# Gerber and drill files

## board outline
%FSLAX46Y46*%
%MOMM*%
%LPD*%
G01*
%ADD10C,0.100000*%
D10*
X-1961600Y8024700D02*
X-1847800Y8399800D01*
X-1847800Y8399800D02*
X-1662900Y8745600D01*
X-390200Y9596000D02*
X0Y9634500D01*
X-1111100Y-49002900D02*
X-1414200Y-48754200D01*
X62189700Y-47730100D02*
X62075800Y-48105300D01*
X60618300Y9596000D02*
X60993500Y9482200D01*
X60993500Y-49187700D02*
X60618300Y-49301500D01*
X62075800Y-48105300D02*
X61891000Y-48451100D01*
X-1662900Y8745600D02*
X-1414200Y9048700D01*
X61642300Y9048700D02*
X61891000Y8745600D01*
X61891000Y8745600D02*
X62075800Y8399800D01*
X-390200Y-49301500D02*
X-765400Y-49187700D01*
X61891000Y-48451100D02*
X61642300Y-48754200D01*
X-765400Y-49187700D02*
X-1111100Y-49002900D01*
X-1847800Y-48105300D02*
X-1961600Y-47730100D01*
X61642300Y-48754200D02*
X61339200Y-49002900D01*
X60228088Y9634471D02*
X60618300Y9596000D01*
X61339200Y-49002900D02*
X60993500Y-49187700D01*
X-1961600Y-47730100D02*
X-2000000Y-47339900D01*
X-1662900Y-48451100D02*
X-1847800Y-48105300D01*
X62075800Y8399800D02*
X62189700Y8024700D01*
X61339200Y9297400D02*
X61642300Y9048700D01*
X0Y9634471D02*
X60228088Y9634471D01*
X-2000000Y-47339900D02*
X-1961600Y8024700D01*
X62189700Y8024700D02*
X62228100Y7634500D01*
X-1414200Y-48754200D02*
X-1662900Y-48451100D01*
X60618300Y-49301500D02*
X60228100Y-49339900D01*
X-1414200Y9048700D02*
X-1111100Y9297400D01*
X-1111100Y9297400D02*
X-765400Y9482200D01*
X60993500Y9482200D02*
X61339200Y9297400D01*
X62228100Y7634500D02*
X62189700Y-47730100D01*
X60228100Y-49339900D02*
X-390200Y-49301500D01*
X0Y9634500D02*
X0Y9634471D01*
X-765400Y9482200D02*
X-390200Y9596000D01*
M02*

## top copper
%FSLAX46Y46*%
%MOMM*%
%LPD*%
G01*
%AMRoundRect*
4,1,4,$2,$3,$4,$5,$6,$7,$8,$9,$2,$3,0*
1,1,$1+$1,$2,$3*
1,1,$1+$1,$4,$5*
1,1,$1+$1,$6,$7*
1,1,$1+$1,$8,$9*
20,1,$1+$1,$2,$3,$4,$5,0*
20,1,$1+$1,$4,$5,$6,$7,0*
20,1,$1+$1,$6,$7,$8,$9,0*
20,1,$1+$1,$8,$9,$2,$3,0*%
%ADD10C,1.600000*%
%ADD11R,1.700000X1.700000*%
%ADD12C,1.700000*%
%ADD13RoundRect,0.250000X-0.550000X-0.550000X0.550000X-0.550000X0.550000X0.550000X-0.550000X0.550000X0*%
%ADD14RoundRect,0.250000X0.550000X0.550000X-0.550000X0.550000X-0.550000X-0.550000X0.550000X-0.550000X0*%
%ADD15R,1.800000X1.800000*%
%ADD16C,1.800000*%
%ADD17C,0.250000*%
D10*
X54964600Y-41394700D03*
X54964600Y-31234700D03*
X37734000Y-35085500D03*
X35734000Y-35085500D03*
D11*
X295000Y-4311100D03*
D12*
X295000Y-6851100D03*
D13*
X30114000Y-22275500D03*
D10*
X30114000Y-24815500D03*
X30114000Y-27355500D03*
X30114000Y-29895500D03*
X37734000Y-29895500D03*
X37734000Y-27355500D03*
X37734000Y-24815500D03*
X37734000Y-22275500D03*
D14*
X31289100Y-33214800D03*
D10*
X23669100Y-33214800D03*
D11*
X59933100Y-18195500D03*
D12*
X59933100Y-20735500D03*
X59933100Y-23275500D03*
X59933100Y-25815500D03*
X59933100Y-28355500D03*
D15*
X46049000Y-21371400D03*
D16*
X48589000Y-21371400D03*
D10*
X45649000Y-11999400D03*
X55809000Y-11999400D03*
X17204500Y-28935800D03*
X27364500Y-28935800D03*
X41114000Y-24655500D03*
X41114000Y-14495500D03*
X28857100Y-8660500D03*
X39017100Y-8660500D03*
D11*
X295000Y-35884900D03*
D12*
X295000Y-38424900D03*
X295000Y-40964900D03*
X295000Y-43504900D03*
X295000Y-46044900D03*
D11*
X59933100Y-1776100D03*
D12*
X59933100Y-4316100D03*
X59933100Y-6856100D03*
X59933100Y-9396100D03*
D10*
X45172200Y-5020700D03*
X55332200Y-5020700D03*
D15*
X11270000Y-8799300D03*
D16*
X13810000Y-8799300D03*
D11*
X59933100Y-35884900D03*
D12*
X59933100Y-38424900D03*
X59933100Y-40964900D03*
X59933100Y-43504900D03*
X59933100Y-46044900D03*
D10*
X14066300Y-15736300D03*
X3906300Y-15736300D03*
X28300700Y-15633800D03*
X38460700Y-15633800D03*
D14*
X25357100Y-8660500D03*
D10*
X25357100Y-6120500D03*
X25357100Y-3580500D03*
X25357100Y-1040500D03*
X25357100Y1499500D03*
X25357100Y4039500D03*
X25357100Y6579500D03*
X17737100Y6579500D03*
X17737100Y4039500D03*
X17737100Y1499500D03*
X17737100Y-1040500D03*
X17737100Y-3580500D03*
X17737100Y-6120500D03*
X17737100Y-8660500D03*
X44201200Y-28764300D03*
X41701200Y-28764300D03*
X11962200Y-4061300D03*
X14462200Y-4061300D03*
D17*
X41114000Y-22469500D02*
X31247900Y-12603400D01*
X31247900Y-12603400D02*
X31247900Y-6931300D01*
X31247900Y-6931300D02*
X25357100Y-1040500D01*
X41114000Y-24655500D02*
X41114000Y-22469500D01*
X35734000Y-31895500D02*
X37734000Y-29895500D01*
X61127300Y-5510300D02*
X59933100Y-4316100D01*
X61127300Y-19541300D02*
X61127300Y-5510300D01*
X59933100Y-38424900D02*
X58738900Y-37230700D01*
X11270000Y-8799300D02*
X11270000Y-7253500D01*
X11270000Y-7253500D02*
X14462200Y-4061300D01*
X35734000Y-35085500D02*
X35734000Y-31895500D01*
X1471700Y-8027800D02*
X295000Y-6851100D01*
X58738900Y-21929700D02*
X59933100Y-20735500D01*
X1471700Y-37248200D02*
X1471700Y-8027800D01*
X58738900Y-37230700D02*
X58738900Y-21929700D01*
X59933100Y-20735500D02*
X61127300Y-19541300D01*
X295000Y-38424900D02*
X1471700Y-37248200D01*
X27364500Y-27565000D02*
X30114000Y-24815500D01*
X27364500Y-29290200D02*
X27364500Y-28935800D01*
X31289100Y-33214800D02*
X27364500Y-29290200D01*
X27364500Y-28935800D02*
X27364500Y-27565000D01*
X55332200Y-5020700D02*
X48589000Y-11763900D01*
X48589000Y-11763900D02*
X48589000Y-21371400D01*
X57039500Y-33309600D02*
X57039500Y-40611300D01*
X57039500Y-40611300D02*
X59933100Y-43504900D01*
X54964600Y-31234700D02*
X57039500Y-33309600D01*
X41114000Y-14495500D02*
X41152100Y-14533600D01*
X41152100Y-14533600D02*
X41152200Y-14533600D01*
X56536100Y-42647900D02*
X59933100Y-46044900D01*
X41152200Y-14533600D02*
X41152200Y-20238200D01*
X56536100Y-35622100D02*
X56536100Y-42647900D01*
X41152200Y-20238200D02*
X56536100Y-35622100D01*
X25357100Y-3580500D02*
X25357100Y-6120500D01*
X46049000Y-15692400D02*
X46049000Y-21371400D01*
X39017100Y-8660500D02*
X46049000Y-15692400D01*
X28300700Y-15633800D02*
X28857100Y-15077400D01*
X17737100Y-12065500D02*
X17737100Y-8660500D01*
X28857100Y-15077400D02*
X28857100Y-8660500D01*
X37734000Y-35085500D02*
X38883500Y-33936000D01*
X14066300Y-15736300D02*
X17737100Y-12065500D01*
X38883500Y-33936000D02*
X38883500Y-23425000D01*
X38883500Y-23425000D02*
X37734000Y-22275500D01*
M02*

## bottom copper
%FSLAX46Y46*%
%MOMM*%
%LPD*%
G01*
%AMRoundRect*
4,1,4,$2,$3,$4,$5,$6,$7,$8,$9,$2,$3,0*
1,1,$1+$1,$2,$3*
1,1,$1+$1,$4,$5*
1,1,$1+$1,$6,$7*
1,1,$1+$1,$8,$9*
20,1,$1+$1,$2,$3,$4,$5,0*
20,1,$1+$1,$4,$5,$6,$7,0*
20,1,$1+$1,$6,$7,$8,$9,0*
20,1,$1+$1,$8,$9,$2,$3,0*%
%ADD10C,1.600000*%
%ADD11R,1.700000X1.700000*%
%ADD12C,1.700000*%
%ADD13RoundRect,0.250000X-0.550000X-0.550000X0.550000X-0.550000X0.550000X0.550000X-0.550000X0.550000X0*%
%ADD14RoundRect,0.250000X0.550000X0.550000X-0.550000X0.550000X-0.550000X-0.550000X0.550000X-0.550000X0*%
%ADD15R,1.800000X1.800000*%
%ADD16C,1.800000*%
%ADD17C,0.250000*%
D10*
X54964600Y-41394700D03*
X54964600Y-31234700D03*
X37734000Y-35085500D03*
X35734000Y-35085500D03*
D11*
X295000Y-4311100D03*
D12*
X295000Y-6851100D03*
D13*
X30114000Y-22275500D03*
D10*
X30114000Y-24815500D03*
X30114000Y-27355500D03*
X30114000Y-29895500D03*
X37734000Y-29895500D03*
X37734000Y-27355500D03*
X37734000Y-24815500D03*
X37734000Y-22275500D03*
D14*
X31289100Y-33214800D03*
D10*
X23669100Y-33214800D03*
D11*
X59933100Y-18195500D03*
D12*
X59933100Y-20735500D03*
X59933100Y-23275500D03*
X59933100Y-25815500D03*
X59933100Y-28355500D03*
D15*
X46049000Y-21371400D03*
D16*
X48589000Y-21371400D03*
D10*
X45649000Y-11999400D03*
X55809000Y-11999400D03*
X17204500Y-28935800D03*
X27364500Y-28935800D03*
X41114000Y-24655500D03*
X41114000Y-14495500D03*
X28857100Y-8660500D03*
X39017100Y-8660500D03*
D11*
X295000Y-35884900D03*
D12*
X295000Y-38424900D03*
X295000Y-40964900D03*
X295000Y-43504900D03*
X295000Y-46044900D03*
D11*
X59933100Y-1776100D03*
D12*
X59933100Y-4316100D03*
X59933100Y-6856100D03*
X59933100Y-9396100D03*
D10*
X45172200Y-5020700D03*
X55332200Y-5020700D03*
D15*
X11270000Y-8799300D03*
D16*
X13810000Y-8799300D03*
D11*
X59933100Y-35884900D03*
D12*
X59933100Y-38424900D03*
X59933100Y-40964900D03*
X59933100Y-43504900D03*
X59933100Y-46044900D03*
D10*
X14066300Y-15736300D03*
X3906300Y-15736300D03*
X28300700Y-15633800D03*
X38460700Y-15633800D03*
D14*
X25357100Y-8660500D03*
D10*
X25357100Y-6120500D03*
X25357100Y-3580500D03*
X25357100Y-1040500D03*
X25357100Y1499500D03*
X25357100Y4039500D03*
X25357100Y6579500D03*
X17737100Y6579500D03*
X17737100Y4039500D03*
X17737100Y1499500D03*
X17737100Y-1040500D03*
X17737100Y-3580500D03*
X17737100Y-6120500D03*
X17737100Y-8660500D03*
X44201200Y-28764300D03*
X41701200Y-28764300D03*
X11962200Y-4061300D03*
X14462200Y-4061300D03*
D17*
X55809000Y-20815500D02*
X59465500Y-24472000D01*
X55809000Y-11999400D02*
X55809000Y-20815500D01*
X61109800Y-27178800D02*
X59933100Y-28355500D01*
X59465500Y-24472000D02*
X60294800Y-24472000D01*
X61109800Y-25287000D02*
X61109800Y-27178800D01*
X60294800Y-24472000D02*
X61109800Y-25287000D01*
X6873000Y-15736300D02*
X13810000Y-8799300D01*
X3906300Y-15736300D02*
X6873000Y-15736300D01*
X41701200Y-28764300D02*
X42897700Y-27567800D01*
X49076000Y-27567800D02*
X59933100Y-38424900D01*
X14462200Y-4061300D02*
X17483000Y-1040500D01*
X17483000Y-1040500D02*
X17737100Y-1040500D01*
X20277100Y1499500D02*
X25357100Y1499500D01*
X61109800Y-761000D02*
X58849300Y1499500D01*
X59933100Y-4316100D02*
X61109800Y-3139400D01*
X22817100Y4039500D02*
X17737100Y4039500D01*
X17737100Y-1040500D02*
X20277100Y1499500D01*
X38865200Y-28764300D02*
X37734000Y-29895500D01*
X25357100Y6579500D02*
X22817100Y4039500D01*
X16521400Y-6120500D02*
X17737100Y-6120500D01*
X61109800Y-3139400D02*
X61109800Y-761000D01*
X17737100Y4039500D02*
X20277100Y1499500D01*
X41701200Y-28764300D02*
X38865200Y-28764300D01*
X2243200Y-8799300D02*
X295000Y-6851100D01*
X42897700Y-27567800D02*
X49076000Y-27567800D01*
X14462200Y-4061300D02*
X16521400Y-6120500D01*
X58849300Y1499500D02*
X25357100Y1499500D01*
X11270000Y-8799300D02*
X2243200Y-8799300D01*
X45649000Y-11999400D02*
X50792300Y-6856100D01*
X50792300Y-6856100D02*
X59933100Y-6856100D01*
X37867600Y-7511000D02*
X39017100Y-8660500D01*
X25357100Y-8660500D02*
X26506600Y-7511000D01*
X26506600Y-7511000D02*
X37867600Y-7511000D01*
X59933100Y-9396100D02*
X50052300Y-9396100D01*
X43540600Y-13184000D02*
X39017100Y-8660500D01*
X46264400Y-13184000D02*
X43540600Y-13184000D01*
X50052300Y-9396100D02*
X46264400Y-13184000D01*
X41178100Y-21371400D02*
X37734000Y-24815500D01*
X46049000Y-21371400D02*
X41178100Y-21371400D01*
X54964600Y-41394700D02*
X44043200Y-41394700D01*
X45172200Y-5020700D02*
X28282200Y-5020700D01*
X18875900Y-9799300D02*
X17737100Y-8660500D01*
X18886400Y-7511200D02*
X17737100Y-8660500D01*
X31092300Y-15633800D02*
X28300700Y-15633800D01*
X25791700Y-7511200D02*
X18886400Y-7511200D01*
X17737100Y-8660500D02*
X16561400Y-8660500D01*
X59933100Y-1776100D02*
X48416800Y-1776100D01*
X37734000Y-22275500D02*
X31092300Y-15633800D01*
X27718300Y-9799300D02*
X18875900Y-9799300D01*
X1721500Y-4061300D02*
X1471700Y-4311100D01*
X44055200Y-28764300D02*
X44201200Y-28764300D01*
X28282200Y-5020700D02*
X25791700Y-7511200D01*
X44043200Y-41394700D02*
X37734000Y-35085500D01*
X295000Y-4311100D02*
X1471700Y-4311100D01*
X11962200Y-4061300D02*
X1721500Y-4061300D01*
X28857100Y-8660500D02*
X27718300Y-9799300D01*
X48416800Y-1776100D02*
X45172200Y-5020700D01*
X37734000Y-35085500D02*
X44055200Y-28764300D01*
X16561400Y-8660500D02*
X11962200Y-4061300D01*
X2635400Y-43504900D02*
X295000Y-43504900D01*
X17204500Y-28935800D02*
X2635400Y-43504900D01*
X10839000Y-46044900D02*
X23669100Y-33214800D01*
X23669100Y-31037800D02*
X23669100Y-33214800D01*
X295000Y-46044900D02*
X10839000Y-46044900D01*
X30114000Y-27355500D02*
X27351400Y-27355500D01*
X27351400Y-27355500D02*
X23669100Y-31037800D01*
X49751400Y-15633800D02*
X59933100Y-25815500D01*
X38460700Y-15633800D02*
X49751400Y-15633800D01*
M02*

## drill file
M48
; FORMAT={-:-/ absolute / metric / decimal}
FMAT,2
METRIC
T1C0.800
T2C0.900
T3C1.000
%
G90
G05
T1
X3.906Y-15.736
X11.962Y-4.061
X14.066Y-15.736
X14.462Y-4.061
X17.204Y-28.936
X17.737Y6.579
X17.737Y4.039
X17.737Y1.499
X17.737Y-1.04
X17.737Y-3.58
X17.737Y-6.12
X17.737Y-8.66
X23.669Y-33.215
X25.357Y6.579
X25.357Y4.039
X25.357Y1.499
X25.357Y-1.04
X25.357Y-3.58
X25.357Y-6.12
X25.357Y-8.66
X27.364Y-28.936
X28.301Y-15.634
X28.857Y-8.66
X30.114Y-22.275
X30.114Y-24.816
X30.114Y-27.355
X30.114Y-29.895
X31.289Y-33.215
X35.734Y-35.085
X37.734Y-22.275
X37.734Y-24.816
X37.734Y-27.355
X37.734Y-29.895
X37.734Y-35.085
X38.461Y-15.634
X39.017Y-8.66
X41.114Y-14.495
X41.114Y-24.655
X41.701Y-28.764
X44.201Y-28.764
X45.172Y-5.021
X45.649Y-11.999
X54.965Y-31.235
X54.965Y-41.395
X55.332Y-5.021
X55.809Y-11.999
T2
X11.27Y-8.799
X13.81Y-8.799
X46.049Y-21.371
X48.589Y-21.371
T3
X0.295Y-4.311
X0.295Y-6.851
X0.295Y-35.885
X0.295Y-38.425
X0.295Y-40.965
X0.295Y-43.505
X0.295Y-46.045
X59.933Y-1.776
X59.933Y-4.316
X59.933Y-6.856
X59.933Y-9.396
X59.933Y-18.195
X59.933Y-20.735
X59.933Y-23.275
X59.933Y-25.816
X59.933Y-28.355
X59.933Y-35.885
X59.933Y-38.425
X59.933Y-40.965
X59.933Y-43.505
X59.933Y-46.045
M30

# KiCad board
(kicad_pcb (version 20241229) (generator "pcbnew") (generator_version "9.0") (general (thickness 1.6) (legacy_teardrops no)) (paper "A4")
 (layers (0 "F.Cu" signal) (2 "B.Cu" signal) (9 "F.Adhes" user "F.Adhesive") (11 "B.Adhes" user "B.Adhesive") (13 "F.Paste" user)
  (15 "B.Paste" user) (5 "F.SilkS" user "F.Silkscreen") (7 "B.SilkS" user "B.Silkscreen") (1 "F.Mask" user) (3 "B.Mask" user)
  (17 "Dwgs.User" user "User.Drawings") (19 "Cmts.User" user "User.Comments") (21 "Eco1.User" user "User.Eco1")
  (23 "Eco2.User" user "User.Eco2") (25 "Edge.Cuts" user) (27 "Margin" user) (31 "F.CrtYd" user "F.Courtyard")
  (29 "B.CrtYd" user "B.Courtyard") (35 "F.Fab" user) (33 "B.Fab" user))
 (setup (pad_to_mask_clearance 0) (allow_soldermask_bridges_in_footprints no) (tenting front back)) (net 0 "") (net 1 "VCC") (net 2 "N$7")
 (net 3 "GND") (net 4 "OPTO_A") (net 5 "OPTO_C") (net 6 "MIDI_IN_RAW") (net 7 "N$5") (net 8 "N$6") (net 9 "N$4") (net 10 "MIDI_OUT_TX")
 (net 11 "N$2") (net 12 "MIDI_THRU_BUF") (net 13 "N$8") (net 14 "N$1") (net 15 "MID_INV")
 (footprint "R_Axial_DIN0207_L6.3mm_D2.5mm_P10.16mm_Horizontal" (layer "F.Cu") (at 54.9646 41.3947 90)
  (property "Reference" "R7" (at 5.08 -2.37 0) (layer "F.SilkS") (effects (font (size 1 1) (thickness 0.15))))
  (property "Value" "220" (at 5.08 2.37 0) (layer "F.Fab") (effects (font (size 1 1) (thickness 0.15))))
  (pad "1" thru_hole circle (at 0 0 90) (size 1.6 1.6) (drill 0.8) (layers "*.Cu" "*.Mask") (remove_unused_layers no) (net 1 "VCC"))
  (pad "2" thru_hole circle (at 10.16 0 90) (size 1.6 1.6) (drill 0.8) (layers "*.Cu" "*.Mask") (remove_unused_layers no) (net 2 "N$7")))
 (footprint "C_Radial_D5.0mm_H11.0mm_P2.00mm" (layer "F.Cu") (at 37.734 35.0855 180)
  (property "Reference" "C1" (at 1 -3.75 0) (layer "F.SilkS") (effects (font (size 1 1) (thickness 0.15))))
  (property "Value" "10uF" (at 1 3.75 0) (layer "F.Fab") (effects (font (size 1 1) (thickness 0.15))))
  (pad "1" thru_hole circle (at 0 0 180) (size 1.6 1.6) (drill 0.8) (layers "*.Cu" "*.Mask") (remove_unused_layers no) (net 1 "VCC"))
  (pad "2" thru_hole circle (at 2 0 180) (size 1.6 1.6) (drill 0.8) (layers "*.Cu" "*.Mask") (remove_unused_layers no) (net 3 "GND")))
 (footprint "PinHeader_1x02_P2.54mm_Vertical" (layer "F.Cu") (at 0.295 4.3111)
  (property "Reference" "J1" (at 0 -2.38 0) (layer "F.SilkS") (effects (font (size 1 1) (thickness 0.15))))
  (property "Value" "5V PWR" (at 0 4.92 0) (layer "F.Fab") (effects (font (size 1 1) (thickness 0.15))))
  (pad "1" thru_hole rect (at 0 0) (size 1.7 1.7) (drill 1) (layers "*.Cu" "*.Mask") (remove_unused_layers no) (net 1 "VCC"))
  (pad "2" thru_hole circle (at 0 2.54) (size 1.7 1.7) (drill 1) (layers "*.Cu" "*.Mask") (remove_unused_layers no) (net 3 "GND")))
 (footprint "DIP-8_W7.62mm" (layer "F.Cu") (at 30.114 22.2755)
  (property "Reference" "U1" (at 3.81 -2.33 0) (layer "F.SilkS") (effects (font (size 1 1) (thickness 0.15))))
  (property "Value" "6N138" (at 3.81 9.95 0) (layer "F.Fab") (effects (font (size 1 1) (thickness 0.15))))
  (pad "1" thru_hole roundrect (at 0 0) (size 1.6 1.6) (drill 0.8) (layers "*.Cu" "*.Mask") (remove_unused_layers no)
   (roundrect_rratio 0.15625))
  (pad "2" thru_hole circle (at 0 2.54) (size 1.6 1.6) (drill 0.8) (layers "*.Cu" "*.Mask") (remove_unused_layers no) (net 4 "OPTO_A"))
  (pad "3" thru_hole circle (at 0 5.08) (size 1.6 1.6) (drill 0.8) (layers "*.Cu" "*.Mask") (remove_unused_layers no) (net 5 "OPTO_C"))
  (pad "4" thru_hole circle (at 0 7.62) (size 1.6 1.6) (drill 0.8) (layers "*.Cu" "*.Mask") (remove_unused_layers no))
  (pad "5" thru_hole circle (at 7.62 7.62) (size 1.6 1.6) (drill 0.8) (layers "*.Cu" "*.Mask") (remove_unused_layers no) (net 3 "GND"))
  (pad "6" thru_hole circle (at 7.62 5.08) (size 1.6 1.6) (drill 0.8) (layers "*.Cu" "*.Mask") (remove_unused_layers no))
  (pad "7" thru_hole circle (at 7.62 2.54) (size 1.6 1.6) (drill 0.8) (layers "*.Cu" "*.Mask") (remove_unused_layers no)
   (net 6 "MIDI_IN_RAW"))
  (pad "8" thru_hole circle (at 7.62 0) (size 1.6 1.6) (drill 0.8) (layers "*.Cu" "*.Mask") (remove_unused_layers no) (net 1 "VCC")))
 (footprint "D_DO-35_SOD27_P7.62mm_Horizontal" (layer "F.Cu") (at 31.2891 33.2148 180)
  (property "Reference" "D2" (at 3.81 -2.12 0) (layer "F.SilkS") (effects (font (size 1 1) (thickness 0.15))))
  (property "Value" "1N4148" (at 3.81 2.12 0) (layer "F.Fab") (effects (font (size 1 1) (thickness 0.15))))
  (pad "1" thru_hole roundrect (at 0 0 180) (size 1.6 1.6) (drill 0.8) (layers "*.Cu" "*.Mask") (remove_unused_layers no)
   (roundrect_rratio 0.15625) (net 4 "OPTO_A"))
  (pad "2" thru_hole circle (at 7.62 0 180) (size 1.6 1.6) (drill 0.8) (layers "*.Cu" "*.Mask") (remove_unused_layers no) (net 5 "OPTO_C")))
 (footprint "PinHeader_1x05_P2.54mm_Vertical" (layer "F.Cu") (at 59.9331 18.1955)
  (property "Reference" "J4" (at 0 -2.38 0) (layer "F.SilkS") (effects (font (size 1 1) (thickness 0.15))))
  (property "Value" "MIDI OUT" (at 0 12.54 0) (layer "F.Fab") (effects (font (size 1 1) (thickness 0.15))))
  (pad "1" thru_hole rect (at 0 0) (size 1.7 1.7) (drill 1) (layers "*.Cu" "*.Mask") (remove_unused_layers no))
  (pad "2" thru_hole circle (at 0 2.54) (size 1.7 1.7) (drill 1) (layers "*.Cu" "*.Mask") (remove_unused_layers no) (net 3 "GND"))
  (pad "3" thru_hole circle (at 0 5.08) (size 1.7 1.7) (drill 1) (layers "*.Cu" "*.Mask") (remove_unused_layers no))
  (pad "4" thru_hole circle (at 0 7.62) (size 1.7 1.7) (drill 1) (layers "*.Cu" "*.Mask") (remove_unused_layers no) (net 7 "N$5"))
  (pad "5" thru_hole circle (at 0 10.16) (size 1.7 1.7) (drill 1) (layers "*.Cu" "*.Mask") (remove_unused_layers no) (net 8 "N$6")))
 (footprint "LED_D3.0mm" (layer "F.Cu") (at 46.049 21.3714)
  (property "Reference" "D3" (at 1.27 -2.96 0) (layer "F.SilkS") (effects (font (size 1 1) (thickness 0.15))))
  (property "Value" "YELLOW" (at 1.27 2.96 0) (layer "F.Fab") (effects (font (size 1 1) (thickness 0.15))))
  (pad "1" thru_hole rect (at 0 0) (size 1.8 1.8) (drill 0.9) (layers "*.Cu" "*.Mask") (remove_unused_layers no) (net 6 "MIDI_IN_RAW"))
  (pad "2" thru_hole circle (at 2.54 0) (size 1.8 1.8) (drill 0.9) (layers "*.Cu" "*.Mask") (remove_unused_layers no) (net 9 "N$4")))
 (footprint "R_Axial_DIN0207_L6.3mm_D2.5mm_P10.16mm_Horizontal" (layer "F.Cu") (at 45.649 11.9994)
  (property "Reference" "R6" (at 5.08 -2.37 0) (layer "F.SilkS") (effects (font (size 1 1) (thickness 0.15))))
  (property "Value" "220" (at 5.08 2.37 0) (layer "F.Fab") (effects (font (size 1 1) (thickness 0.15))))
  (pad "1" thru_hole circle (at 0 0) (size 1.6 1.6) (drill 0.8) (layers "*.Cu" "*.Mask") (remove_unused_layers no) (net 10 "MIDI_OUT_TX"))
  (pad "2" thru_hole circle (at 10.16 0) (size 1.6 1.6) (drill 0.8) (layers "*.Cu" "*.Mask") (remove_unused_layers no) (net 8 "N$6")))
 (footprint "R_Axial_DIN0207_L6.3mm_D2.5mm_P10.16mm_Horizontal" (layer "F.Cu") (at 17.2045 28.9358)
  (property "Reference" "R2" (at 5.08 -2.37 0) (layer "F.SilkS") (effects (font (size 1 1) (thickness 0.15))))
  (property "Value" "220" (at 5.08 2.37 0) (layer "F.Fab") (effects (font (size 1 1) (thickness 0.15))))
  (pad "1" thru_hole circle (at 0 0) (size 1.6 1.6) (drill 0.8) (layers "*.Cu" "*.Mask") (remove_unused_layers no) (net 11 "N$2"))
  (pad "2" thru_hole circle (at 10.16 0) (size 1.6 1.6) (drill 0.8) (layers "*.Cu" "*.Mask") (remove_unused_layers no) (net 4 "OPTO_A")))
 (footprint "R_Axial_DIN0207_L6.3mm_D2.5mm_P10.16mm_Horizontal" (layer "F.Cu") (at 41.114 24.6555 90)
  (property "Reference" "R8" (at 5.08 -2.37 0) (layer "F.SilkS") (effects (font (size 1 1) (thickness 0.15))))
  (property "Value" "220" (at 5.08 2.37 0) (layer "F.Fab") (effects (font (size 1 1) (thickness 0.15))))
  (pad "1" thru_hole circle (at 0 0 90) (size 1.6 1.6) (drill 0.8) (layers "*.Cu" "*.Mask") (remove_unused_layers no)
   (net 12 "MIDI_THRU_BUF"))
  (pad "2" thru_hole circle (at 10.16 0 90) (size 1.6 1.6) (drill 0.8) (layers "*.Cu" "*.Mask") (remove_unused_layers no) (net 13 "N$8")))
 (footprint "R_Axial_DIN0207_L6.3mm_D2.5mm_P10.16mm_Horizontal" (layer "F.Cu") (at 28.8571 8.6605)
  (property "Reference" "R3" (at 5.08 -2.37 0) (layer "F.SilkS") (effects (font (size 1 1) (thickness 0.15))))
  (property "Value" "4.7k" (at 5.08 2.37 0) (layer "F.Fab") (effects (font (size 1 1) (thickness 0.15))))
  (pad "1" thru_hole circle (at 0 0) (size 1.6 1.6) (drill 0.8) (layers "*.Cu" "*.Mask") (remove_unused_layers no) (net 1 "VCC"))
  (pad "2" thru_hole circle (at 10.16 0) (size 1.6 1.6) (drill 0.8) (layers "*.Cu" "*.Mask") (remove_unused_layers no) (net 6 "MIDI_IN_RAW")))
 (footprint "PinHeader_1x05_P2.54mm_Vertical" (layer "F.Cu") (at 0.295 35.8849)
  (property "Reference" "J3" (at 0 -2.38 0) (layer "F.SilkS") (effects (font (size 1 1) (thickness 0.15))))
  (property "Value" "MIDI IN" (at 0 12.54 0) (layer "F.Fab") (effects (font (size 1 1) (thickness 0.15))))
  (pad "1" thru_hole rect (at 0 0) (size 1.7 1.7) (drill 1) (layers "*.Cu" "*.Mask") (remove_unused_layers no))
  (pad "2" thru_hole circle (at 0 2.54) (size 1.7 1.7) (drill 1) (layers "*.Cu" "*.Mask") (remove_unused_layers no) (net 3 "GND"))
  (pad "3" thru_hole circle (at 0 5.08) (size 1.7 1.7) (drill 1) (layers "*.Cu" "*.Mask") (remove_unused_layers no))
  (pad "4" thru_hole circle (at 0 7.62) (size 1.7 1.7) (drill 1) (layers "*.Cu" "*.Mask") (remove_unused_layers no) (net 11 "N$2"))
  (pad "5" thru_hole circle (at 0 10.16) (size 1.7 1.7) (drill 1) (layers "*.Cu" "*.Mask") (remove_unused_layers no) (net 5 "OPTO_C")))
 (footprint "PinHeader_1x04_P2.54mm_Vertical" (layer "F.Cu") (at 59.9331 1.7761)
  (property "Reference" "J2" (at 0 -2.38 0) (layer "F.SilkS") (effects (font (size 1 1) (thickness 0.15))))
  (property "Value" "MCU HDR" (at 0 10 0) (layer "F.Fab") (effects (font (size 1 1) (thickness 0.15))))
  (pad "1" thru_hole rect (at 0 0) (size 1.7 1.7) (drill 1) (layers "*.Cu" "*.Mask") (remove_unused_layers no) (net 1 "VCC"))
  (pad "2" thru_hole circle (at 0 2.54) (size 1.7 1.7) (drill 1) (layers "*.Cu" "*.Mask") (remove_unused_layers no) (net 3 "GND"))
  (pad "3" thru_hole circle (at 0 5.08) (size 1.7 1.7) (drill 1) (layers "*.Cu" "*.Mask") (remove_unused_layers no) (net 10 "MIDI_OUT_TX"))
  (pad "4" thru_hole circle (at 0 7.62) (size 1.7 1.7) (drill 1) (layers "*.Cu" "*.Mask") (remove_unused_layers no) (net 6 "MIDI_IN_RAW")))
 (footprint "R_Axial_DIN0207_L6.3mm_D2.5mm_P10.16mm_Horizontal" (layer "F.Cu") (at 45.1722 5.0207)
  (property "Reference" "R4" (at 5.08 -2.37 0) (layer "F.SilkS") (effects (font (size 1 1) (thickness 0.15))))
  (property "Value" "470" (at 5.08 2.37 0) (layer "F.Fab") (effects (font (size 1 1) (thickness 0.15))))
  (pad "1" thru_hole circle (at 0 0) (size 1.6 1.6) (drill 0.8) (layers "*.Cu" "*.Mask") (remove_unused_layers no) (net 1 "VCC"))
  (pad "2" thru_hole circle (at 10.16 0) (size 1.6 1.6) (drill 0.8) (layers "*.Cu" "*.Mask") (remove_unused_layers no) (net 9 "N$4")))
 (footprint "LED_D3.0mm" (layer "F.Cu") (at 11.27 8.7993)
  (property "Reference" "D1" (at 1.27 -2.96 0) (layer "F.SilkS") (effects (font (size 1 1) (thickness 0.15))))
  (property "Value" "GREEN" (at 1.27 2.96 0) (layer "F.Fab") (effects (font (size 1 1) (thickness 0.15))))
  (pad "1" thru_hole rect (at 0 0) (size 1.8 1.8) (drill 0.9) (layers "*.Cu" "*.Mask") (remove_unused_layers no) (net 3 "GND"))
  (pad "2" thru_hole circle (at 2.54 0) (size 1.8 1.8) (drill 0.9) (layers "*.Cu" "*.Mask") (remove_unused_layers no) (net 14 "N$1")))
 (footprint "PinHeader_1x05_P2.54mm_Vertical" (layer "F.Cu") (at 59.9331 35.8849)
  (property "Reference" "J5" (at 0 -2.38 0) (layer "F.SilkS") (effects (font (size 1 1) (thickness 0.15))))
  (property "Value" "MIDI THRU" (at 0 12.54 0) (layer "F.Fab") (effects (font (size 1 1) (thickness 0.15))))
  (pad "1" thru_hole rect (at 0 0) (size 1.7 1.7) (drill 1) (layers "*.Cu" "*.Mask") (remove_unused_layers no))
  (pad "2" thru_hole circle (at 0 2.54) (size 1.7 1.7) (drill 1) (layers "*.Cu" "*.Mask") (remove_unused_layers no) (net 3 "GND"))
  (pad "3" thru_hole circle (at 0 5.08) (size 1.7 1.7) (drill 1) (layers "*.Cu" "*.Mask") (remove_unused_layers no))
  (pad "4" thru_hole circle (at 0 7.62) (size 1.7 1.7) (drill 1) (layers "*.Cu" "*.Mask") (remove_unused_layers no) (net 2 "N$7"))
  (pad "5" thru_hole circle (at 0 10.16) (size 1.7 1.7) (drill 1) (layers "*.Cu" "*.Mask") (remove_unused_layers no) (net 13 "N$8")))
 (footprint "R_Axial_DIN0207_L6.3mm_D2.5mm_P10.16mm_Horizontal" (layer "F.Cu") (at 14.0663 15.7363 180)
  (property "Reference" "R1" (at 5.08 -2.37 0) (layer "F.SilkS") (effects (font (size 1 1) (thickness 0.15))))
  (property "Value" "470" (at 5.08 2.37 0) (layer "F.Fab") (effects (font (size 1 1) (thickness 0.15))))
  (pad "1" thru_hole circle (at 0 0 180) (size 1.6 1.6) (drill 0.8) (layers "*.Cu" "*.Mask") (remove_unused_layers no) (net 1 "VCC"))
  (pad "2" thru_hole circle (at 10.16 0 180) (size 1.6 1.6) (drill 0.8) (layers "*.Cu" "*.Mask") (remove_unused_layers no) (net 14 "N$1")))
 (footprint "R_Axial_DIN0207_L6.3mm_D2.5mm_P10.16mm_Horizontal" (layer "F.Cu") (at 28.3007 15.6338)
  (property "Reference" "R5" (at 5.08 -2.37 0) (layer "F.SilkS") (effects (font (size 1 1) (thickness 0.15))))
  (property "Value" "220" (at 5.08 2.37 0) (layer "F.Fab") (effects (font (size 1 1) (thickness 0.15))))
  (pad "1" thru_hole circle (at 0 0) (size 1.6 1.6) (drill 0.8) (layers "*.Cu" "*.Mask") (remove_unused_layers no) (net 1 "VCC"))
  (pad "2" thru_hole circle (at 10.16 0) (size 1.6 1.6) (drill 0.8) (layers "*.Cu" "*.Mask") (remove_unused_layers no) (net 7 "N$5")))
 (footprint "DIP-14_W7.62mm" (layer "F.Cu") (at 25.3571 8.6605 180)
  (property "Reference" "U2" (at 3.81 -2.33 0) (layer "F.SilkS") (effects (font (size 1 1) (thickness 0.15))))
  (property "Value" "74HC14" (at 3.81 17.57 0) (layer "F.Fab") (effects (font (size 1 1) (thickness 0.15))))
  (pad "1" thru_hole roundrect (at 0 0 180) (size 1.6 1.6) (drill 0.8) (layers "*.Cu" "*.Mask") (remove_unused_layers no)
   (roundrect_rratio 0.15625) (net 6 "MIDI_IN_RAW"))
  (pad "2" thru_hole circle (at 0 2.54 180) (size 1.6 1.6) (drill 0.8) (layers "*.Cu" "*.Mask") (remove_unused_layers no) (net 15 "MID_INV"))
  (pad "3" thru_hole circle (at 0 5.08 180) (size 1.6 1.6) (drill 0.8) (layers "*.Cu" "*.Mask") (remove_unused_layers no) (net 15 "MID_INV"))
  (pad "4" thru_hole circle (at 0 7.62 180) (size 1.6 1.6) (drill 0.8) (layers "*.Cu" "*.Mask") (remove_unused_layers no)
   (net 12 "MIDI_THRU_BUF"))
  (pad "5" thru_hole circle (at 0 10.16 180) (size 1.6 1.6) (drill 0.8) (layers "*.Cu" "*.Mask") (remove_unused_layers no) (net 3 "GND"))
  (pad "6" thru_hole circle (at 0 12.7 180) (size 1.6 1.6) (drill 0.8) (layers "*.Cu" "*.Mask") (remove_unused_layers no))
  (pad "7" thru_hole circle (at 0 15.24 180) (size 1.6 1.6) (drill 0.8) (layers "*.Cu" "*.Mask") (remove_unused_layers no) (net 3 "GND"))
  (pad "8" thru_hole circle (at 7.62 15.24 180) (size 1.6 1.6) (drill 0.8) (layers "*.Cu" "*.Mask") (remove_unused_layers no))
  (pad "9" thru_hole circle (at 7.62 12.7 180) (size 1.6 1.6) (drill 0.8) (layers "*.Cu" "*.Mask") (remove_unused_layers no) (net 3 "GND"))
  (pad "10" thru_hole circle (at 7.62 10.16 180) (size 1.6 1.6) (drill 0.8) (layers "*.Cu" "*.Mask") (remove_unused_layers no))
  (pad "11" thru_hole circle (at 7.62 7.62 180) (size 1.6 1.6) (drill 0.8) (layers "*.Cu" "*.Mask") (remove_unused_layers no) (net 3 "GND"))
  (pad "12" thru_hole circle (at 7.62 5.08 180) (size 1.6 1.6) (drill 0.8) (layers "*.Cu" "*.Mask") (remove_unused_layers no))
  (pad "13" thru_hole circle (at 7.62 2.54 180) (size 1.6 1.6) (drill 0.8) (layers "*.Cu" "*.Mask") (remove_unused_layers no) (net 3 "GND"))
  (pad "14" thru_hole circle (at 7.62 0 180) (size 1.6 1.6) (drill 0.8) (layers "*.Cu" "*.Mask") (remove_unused_layers no) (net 1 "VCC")))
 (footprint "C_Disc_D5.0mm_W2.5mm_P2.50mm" (layer "F.Cu") (at 44.2012 28.7643 180)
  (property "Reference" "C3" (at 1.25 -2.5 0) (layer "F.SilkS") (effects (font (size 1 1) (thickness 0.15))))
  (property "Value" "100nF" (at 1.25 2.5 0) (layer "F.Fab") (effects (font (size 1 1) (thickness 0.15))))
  (pad "1" thru_hole circle (at 0 0 180) (size 1.6 1.6) (drill 0.8) (layers "*.Cu" "*.Mask") (remove_unused_layers no) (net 1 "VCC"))
  (pad "2" thru_hole circle (at 2.5 0 180) (size 1.6 1.6) (drill 0.8) (layers "*.Cu" "*.Mask") (remove_unused_layers no) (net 3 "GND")))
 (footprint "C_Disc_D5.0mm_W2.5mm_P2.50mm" (layer "F.Cu") (at 11.9622 4.0613)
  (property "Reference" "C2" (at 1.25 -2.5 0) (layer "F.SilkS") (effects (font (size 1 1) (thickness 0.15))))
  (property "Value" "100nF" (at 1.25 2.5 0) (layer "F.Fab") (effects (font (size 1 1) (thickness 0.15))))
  (pad "1" thru_hole circle (at 0 0) (size 1.6 1.6) (drill 0.8) (layers "*.Cu" "*.Mask") (remove_unused_layers no) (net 1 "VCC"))
  (pad "2" thru_hole circle (at 2.5 0) (size 1.6 1.6) (drill 0.8) (layers "*.Cu" "*.Mask") (remove_unused_layers no) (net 3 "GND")))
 (gr_line (start -1.9616 -8.0247) (end -1.8478 -8.3998) (stroke (width 0.1) (type solid)) (layer "Edge.Cuts"))
 (gr_line (start -1.8478 -8.3998) (end -1.6629 -8.7456) (stroke (width 0.1) (type solid)) (layer "Edge.Cuts"))
 (gr_line (start -0.3902 -9.596) (end 0 -9.6345) (stroke (width 0.1) (type solid)) (layer "Edge.Cuts"))
 (gr_line (start -1.1111 49.0029) (end -1.4142 48.7542) (stroke (width 0.1) (type solid)) (layer "Edge.Cuts"))
 (gr_line (start 62.1897 47.7301) (end 62.0758 48.1053) (stroke (width 0.1) (type solid)) (layer "Edge.Cuts"))
 (gr_line (start 60.6183 -9.596) (end 60.9935 -9.4822) (stroke (width 0.1) (type solid)) (layer "Edge.Cuts"))
 (gr_line (start 60.9935 49.1877) (end 60.6183 49.3015) (stroke (width 0.1) (type solid)) (layer "Edge.Cuts"))
 (gr_line (start 62.0758 48.1053) (end 61.891 48.4511) (stroke (width 0.1) (type solid)) (layer "Edge.Cuts"))
 (gr_line (start -1.6629 -8.7456) (end -1.4142 -9.0487) (stroke (width 0.1) (type solid)) (layer "Edge.Cuts"))
 (gr_line (start 61.6423 -9.0487) (end 61.891 -8.7456) (stroke (width 0.1) (type solid)) (layer "Edge.Cuts"))
 (gr_line (start 61.891 -8.7456) (end 62.0758 -8.3998) (stroke (width 0.1) (type solid)) (layer "Edge.Cuts"))
 (gr_line (start -0.3902 49.3015) (end -0.7654 49.1877) (stroke (width 0.1) (type solid)) (layer "Edge.Cuts"))
 (gr_line (start 61.891 48.4511) (end 61.6423 48.7542) (stroke (width 0.1) (type solid)) (layer "Edge.Cuts"))
 (gr_line (start -0.7654 49.1877) (end -1.1111 49.0029) (stroke (width 0.1) (type solid)) (layer "Edge.Cuts"))
 (gr_line (start -1.8478 48.1053) (end -1.9616 47.7301) (stroke (width 0.1) (type solid)) (layer "Edge.Cuts"))
 (gr_line (start 61.6423 48.7542) (end 61.3392 49.0029) (stroke (width 0.1) (type solid)) (layer "Edge.Cuts"))
 (gr_line (start 60.228088 -9.634471) (end 60.6183 -9.596) (stroke (width 0.1) (type solid)) (layer "Edge.Cuts"))
 (gr_line (start 61.3392 49.0029) (end 60.9935 49.1877) (stroke (width 0.1) (type solid)) (layer "Edge.Cuts"))
 (gr_line (start -1.9616 47.7301) (end -2 47.3399) (stroke (width 0.1) (type solid)) (layer "Edge.Cuts"))
 (gr_line (start -1.6629 48.4511) (end -1.8478 48.1053) (stroke (width 0.1) (type solid)) (layer "Edge.Cuts"))
 (gr_line (start 62.0758 -8.3998) (end 62.1897 -8.0247) (stroke (width 0.1) (type solid)) (layer "Edge.Cuts"))
 (gr_line (start 61.3392 -9.2974) (end 61.6423 -9.0487) (stroke (width 0.1) (type solid)) (layer "Edge.Cuts"))
 (gr_line (start 0 -9.634471) (end 60.228088 -9.634471) (stroke (width 0.1) (type solid)) (layer "Edge.Cuts"))
 (gr_line (start -2 47.3399) (end -1.9616 -8.0247) (stroke (width 0.1) (type solid)) (layer "Edge.Cuts"))
 (gr_line (start 62.1897 -8.0247) (end 62.2281 -7.6345) (stroke (width 0.1) (type solid)) (layer "Edge.Cuts"))
 (gr_line (start -1.4142 48.7542) (end -1.6629 48.4511) (stroke (width 0.1) (type solid)) (layer "Edge.Cuts"))
 (gr_line (start 60.6183 49.3015) (end 60.2281 49.3399) (stroke (width 0.1) (type solid)) (layer "Edge.Cuts"))
 (gr_line (start -1.4142 -9.0487) (end -1.1111 -9.2974) (stroke (width 0.1) (type solid)) (layer "Edge.Cuts"))
 (gr_line (start -1.1111 -9.2974) (end -0.7654 -9.4822) (stroke (width 0.1) (type solid)) (layer "Edge.Cuts"))
 (gr_line (start 60.9935 -9.4822) (end 61.3392 -9.2974) (stroke (width 0.1) (type solid)) (layer "Edge.Cuts"))
 (gr_line (start 62.2281 -7.6345) (end 62.1897 47.7301) (stroke (width 0.1) (type solid)) (layer "Edge.Cuts"))
 (gr_line (start 60.2281 49.3399) (end -0.3902 49.3015) (stroke (width 0.1) (type solid)) (layer "Edge.Cuts"))
 (gr_line (start 0 -9.6345) (end 0 -9.634471) (stroke (width 0.1) (type solid)) (layer "Edge.Cuts"))
 (gr_line (start -0.7654 -9.4822) (end -0.3902 -9.596) (stroke (width 0.1) (type solid)) (layer "Edge.Cuts"))
 (segment (start 55.809 20.8155) (end 59.4655 24.472) (width 0.25) (layer "B.Cu") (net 8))
 (segment (start 55.809 11.9994) (end 55.809 20.8155) (width 0.25) (layer "B.Cu") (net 8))
 (segment (start 61.1098 27.1788) (end 59.9331 28.3555) (width 0.25) (layer "B.Cu") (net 8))
 (segment (start 59.4655 24.472) (end 60.2948 24.472) (width 0.25) (layer "B.Cu") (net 8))
 (segment (start 61.1098 25.287) (end 61.1098 27.1788) (width 0.25) (layer "B.Cu") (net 8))
 (segment (start 60.2948 24.472) (end 61.1098 25.287) (width 0.25) (layer "B.Cu") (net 8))
 (segment (start 41.114 22.4695) (end 31.2479 12.6034) (width 0.25) (layer "F.Cu") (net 12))
 (segment (start 31.2479 12.6034) (end 31.2479 6.9313) (width 0.25) (layer "F.Cu") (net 12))
 (segment (start 31.2479 6.9313) (end 25.3571 1.0405) (width 0.25) (layer "F.Cu") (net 12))
 (segment (start 41.114 24.6555) (end 41.114 22.4695) (width 0.25) (layer "F.Cu") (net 12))
 (segment (start 6.873 15.7363) (end 13.81 8.7993) (width 0.25) (layer "B.Cu") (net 14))
 (segment (start 3.9063 15.7363) (end 6.873 15.7363) (width 0.25) (layer "B.Cu") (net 14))
 (segment (start 35.734 31.8955) (end 37.734 29.8955) (width 0.25) (layer "F.Cu") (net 3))
 (segment (start 61.1273 5.5103) (end 59.9331 4.3161) (width 0.25) (layer "F.Cu") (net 3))
 (segment (start 61.1273 19.5413) (end 61.1273 5.5103) (width 0.25) (layer "F.Cu") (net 3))
 (segment (start 59.9331 38.4249) (end 58.7389 37.2307) (width 0.25) (layer "F.Cu") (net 3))
 (segment (start 11.27 8.7993) (end 11.27 7.2535) (width 0.25) (layer "F.Cu") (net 3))
 (segment (start 11.27 7.2535) (end 14.4622 4.0613) (width 0.25) (layer "F.Cu") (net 3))
 (segment (start 35.734 35.0855) (end 35.734 31.8955) (width 0.25) (layer "F.Cu") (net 3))
 (segment (start 1.4717 8.0278) (end 0.295 6.8511) (width 0.25) (layer "F.Cu") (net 3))
 (segment (start 58.7389 21.9297) (end 59.9331 20.7355) (width 0.25) (layer "F.Cu") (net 3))
 (segment (start 1.4717 37.2482) (end 1.4717 8.0278) (width 0.25) (layer "F.Cu") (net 3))
 (segment (start 58.7389 37.2307) (end 58.7389 21.9297) (width 0.25) (layer "F.Cu") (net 3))
 (segment (start 59.9331 20.7355) (end 61.1273 19.5413) (width 0.25) (layer "F.Cu") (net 3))
 (segment (start 0.295 38.4249) (end 1.4717 37.2482) (width 0.25) (layer "F.Cu") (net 3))
 (segment (start 41.7012 28.7643) (end 42.8977 27.5678) (width 0.25) (layer "B.Cu") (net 3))
 (segment (start 49.076 27.5678) (end 59.9331 38.4249) (width 0.25) (layer "B.Cu") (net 3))
 (segment (start 14.4622 4.0613) (end 17.483 1.0405) (width 0.25) (layer "B.Cu") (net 3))
 (segment (start 17.483 1.0405) (end 17.7371 1.0405) (width 0.25) (layer "B.Cu") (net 3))
 (segment (start 20.2771 -1.4995) (end 25.3571 -1.4995) (width 0.25) (layer "B.Cu") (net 3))
 (segment (start 61.1098 0.761) (end 58.8493 -1.4995) (width 0.25) (layer "B.Cu") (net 3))
 (segment (start 59.9331 4.3161) (end 61.1098 3.1394) (width 0.25) (layer "B.Cu") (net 3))
 (segment (start 22.8171 -4.0395) (end 17.7371 -4.0395) (width 0.25) (layer "B.Cu") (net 3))
 (segment (start 17.7371 1.0405) (end 20.2771 -1.4995) (width 0.25) (layer "B.Cu") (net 3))
 (segment (start 38.8652 28.7643) (end 37.734 29.8955) (width 0.25) (layer "B.Cu") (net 3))
 (segment (start 25.3571 -6.5795) (end 22.8171 -4.0395) (width 0.25) (layer "B.Cu") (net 3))
 (segment (start 16.5214 6.1205) (end 17.7371 6.1205) (width 0.25) (layer "B.Cu") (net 3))
 (segment (start 61.1098 3.1394) (end 61.1098 0.761) (width 0.25) (layer "B.Cu") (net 3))
 (segment (start 17.7371 -4.0395) (end 20.2771 -1.4995) (width 0.25) (layer "B.Cu") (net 3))
 (segment (start 41.7012 28.7643) (end 38.8652 28.7643) (width 0.25) (layer "B.Cu") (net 3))
 (segment (start 2.2432 8.7993) (end 0.295 6.8511) (width 0.25) (layer "B.Cu") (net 3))
 (segment (start 42.8977 27.5678) (end 49.076 27.5678) (width 0.25) (layer "B.Cu") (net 3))
 (segment (start 14.4622 4.0613) (end 16.5214 6.1205) (width 0.25) (layer "B.Cu") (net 3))
 (segment (start 58.8493 -1.4995) (end 25.3571 -1.4995) (width 0.25) (layer "B.Cu") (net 3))
 (segment (start 11.27 8.7993) (end 2.2432 8.7993) (width 0.25) (layer "B.Cu") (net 3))
 (segment (start 27.3645 27.565) (end 30.114 24.8155) (width 0.25) (layer "F.Cu") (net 4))
 (segment (start 27.3645 29.2902) (end 27.3645 28.9358) (width 0.25) (layer "F.Cu") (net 4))
 (segment (start 31.2891 33.2148) (end 27.3645 29.2902) (width 0.25) (layer "F.Cu") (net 4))
 (segment (start 27.3645 28.9358) (end 27.3645 27.565) (width 0.25) (layer "F.Cu") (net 4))
 (segment (start 55.3322 5.0207) (end 48.589 11.7639) (width 0.25) (layer "F.Cu") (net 9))
 (segment (start 48.589 11.7639) (end 48.589 21.3714) (width 0.25) (layer "F.Cu") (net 9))
 (segment (start 57.0395 33.3096) (end 57.0395 40.6113) (width 0.25) (layer "F.Cu") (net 2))
 (segment (start 57.0395 40.6113) (end 59.9331 43.5049) (width 0.25) (layer "F.Cu") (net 2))
 (segment (start 54.9646 31.2347) (end 57.0395 33.3096) (width 0.25) (layer "F.Cu") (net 2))
 (segment (start 41.114 14.4955) (end 41.1521 14.5336) (width 0.25) (layer "F.Cu") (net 13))
 (segment (start 41.1521 14.5336) (end 41.1522 14.5336) (width 0.25) (layer "F.Cu") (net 13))
 (segment (start 56.5361 42.6479) (end 59.9331 46.0449) (width 0.25) (layer "F.Cu") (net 13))
 (segment (start 41.1522 14.5336) (end 41.1522 20.2382) (width 0.25) (layer "F.Cu") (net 13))
 (segment (start 56.5361 35.6221) (end 56.5361 42.6479) (width 0.25) (layer "F.Cu") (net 13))
 (segment (start 41.1522 20.2382) (end 56.5361 35.6221) (width 0.25) (layer "F.Cu") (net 13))
 (segment (start 25.3571 3.5805) (end 25.3571 6.1205) (width 0.25) (layer "F.Cu") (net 15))
 (segment (start 45.649 11.9994) (end 50.7923 6.8561) (width 0.25) (layer "B.Cu") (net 10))
 (segment (start 50.7923 6.8561) (end 59.9331 6.8561) (width 0.25) (layer "B.Cu") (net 10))
 (segment (start 46.049 15.6924) (end 46.049 21.3714) (width 0.25) (layer "F.Cu") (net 6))
 (segment (start 39.0171 8.6605) (end 46.049 15.6924) (width 0.25) (layer "F.Cu") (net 6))
 (segment (start 37.8676 7.511) (end 39.0171 8.6605) (width 0.25) (layer "B.Cu") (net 6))
 (segment (start 25.3571 8.6605) (end 26.5066 7.511) (width 0.25) (layer "B.Cu") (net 6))
 (segment (start 26.5066 7.511) (end 37.8676 7.511) (width 0.25) (layer "B.Cu") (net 6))
 (segment (start 59.9331 9.3961) (end 50.0523 9.3961) (width 0.25) (layer "B.Cu") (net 6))
 (segment (start 43.5406 13.184) (end 39.0171 8.6605) (width 0.25) (layer "B.Cu") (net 6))
 (segment (start 46.2644 13.184) (end 43.5406 13.184) (width 0.25) (layer "B.Cu") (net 6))
 (segment (start 50.0523 9.3961) (end 46.2644 13.184) (width 0.25) (layer "B.Cu") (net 6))
 (segment (start 41.1781 21.3714) (end 37.734 24.8155) (width 0.25) (layer "B.Cu") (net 6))
 (segment (start 46.049 21.3714) (end 41.1781 21.3714) (width 0.25) (layer "B.Cu") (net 6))
 (segment (start 28.3007 15.6338) (end 28.8571 15.0774) (width 0.25) (layer "F.Cu") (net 1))
 (segment (start 17.7371 12.0655) (end 17.7371 8.6605) (width 0.25) (layer "F.Cu") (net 1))
 (segment (start 28.8571 15.0774) (end 28.8571 8.6605) (width 0.25) (layer "F.Cu") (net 1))
 (segment (start 37.734 35.0855) (end 38.8835 33.936) (width 0.25) (layer "F.Cu") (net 1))
 (segment (start 14.0663 15.7363) (end 17.7371 12.0655) (width 0.25) (layer "F.Cu") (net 1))
 (segment (start 38.8835 33.936) (end 38.8835 23.425) (width 0.25) (layer "F.Cu") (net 1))
 (segment (start 38.8835 23.425) (end 37.734 22.2755) (width 0.25) (layer "F.Cu") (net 1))
 (segment (start 54.9646 41.3947) (end 44.0432 41.3947) (width 0.25) (layer "B.Cu") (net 1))
 (segment (start 45.1722 5.0207) (end 28.2822 5.0207) (width 0.25) (layer "B.Cu") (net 1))
 (segment (start 18.8759 9.7993) (end 17.7371 8.6605) (width 0.25) (layer "B.Cu") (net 1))
 (segment (start 18.8864 7.5112) (end 17.7371 8.6605) (width 0.25) (layer "B.Cu") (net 1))
 (segment (start 31.0923 15.6338) (end 28.3007 15.6338) (width 0.25) (layer "B.Cu") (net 1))
 (segment (start 25.7917 7.5112) (end 18.8864 7.5112) (width 0.25) (layer "B.Cu") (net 1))
 (segment (start 17.7371 8.6605) (end 16.5614 8.6605) (width 0.25) (layer "B.Cu") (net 1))
 (segment (start 59.9331 1.7761) (end 48.4168 1.7761) (width 0.25) (layer "B.Cu") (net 1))
 (segment (start 37.734 22.2755) (end 31.0923 15.6338) (width 0.25) (layer "B.Cu") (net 1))
 (segment (start 27.7183 9.7993) (end 18.8759 9.7993) (width 0.25) (layer "B.Cu") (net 1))
 (segment (start 1.7215 4.0613) (end 1.4717 4.3111) (width 0.25) (layer "B.Cu") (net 1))
 (segment (start 44.0552 28.7643) (end 44.2012 28.7643) (width 0.25) (layer "B.Cu") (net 1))
 (segment (start 28.2822 5.0207) (end 25.7917 7.5112) (width 0.25) (layer "B.Cu") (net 1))
 (segment (start 44.0432 41.3947) (end 37.734 35.0855) (width 0.25) (layer "B.Cu") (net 1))
 (segment (start 0.295 4.3111) (end 1.4717 4.3111) (width 0.25) (layer "B.Cu") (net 1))
 (segment (start 11.9622 4.0613) (end 1.7215 4.0613) (width 0.25) (layer "B.Cu") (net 1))
 (segment (start 28.8571 8.6605) (end 27.7183 9.7993) (width 0.25) (layer "B.Cu") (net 1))
 (segment (start 48.4168 1.7761) (end 45.1722 5.0207) (width 0.25) (layer "B.Cu") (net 1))
 (segment (start 37.734 35.0855) (end 44.0552 28.7643) (width 0.25) (layer "B.Cu") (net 1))
 (segment (start 16.5614 8.6605) (end 11.9622 4.0613) (width 0.25) (layer "B.Cu") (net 1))
 (segment (start 2.6354 43.5049) (end 0.295 43.5049) (width 0.25) (layer "B.Cu") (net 11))
 (segment (start 17.2045 28.9358) (end 2.6354 43.5049) (width 0.25) (layer "B.Cu") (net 11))
 (segment (start 10.839 46.0449) (end 23.6691 33.2148) (width 0.25) (layer "B.Cu") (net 5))
 (segment (start 23.6691 31.0378) (end 23.6691 33.2148) (width 0.25) (layer "B.Cu") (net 5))
 (segment (start 0.295 46.0449) (end 10.839 46.0449) (width 0.25) (layer "B.Cu") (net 5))
 (segment (start 30.114 27.3555) (end 27.3514 27.3555) (width 0.25) (layer "B.Cu") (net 5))
 (segment (start 27.3514 27.3555) (end 23.6691 31.0378) (width 0.25) (layer "B.Cu") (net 5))
 (segment (start 49.7514 15.6338) (end 59.9331 25.8155) (width 0.25) (layer "B.Cu") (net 7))
 (segment (start 38.4607 15.6338) (end 49.7514 15.6338) (width 0.25) (layer "B.Cu") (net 7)))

